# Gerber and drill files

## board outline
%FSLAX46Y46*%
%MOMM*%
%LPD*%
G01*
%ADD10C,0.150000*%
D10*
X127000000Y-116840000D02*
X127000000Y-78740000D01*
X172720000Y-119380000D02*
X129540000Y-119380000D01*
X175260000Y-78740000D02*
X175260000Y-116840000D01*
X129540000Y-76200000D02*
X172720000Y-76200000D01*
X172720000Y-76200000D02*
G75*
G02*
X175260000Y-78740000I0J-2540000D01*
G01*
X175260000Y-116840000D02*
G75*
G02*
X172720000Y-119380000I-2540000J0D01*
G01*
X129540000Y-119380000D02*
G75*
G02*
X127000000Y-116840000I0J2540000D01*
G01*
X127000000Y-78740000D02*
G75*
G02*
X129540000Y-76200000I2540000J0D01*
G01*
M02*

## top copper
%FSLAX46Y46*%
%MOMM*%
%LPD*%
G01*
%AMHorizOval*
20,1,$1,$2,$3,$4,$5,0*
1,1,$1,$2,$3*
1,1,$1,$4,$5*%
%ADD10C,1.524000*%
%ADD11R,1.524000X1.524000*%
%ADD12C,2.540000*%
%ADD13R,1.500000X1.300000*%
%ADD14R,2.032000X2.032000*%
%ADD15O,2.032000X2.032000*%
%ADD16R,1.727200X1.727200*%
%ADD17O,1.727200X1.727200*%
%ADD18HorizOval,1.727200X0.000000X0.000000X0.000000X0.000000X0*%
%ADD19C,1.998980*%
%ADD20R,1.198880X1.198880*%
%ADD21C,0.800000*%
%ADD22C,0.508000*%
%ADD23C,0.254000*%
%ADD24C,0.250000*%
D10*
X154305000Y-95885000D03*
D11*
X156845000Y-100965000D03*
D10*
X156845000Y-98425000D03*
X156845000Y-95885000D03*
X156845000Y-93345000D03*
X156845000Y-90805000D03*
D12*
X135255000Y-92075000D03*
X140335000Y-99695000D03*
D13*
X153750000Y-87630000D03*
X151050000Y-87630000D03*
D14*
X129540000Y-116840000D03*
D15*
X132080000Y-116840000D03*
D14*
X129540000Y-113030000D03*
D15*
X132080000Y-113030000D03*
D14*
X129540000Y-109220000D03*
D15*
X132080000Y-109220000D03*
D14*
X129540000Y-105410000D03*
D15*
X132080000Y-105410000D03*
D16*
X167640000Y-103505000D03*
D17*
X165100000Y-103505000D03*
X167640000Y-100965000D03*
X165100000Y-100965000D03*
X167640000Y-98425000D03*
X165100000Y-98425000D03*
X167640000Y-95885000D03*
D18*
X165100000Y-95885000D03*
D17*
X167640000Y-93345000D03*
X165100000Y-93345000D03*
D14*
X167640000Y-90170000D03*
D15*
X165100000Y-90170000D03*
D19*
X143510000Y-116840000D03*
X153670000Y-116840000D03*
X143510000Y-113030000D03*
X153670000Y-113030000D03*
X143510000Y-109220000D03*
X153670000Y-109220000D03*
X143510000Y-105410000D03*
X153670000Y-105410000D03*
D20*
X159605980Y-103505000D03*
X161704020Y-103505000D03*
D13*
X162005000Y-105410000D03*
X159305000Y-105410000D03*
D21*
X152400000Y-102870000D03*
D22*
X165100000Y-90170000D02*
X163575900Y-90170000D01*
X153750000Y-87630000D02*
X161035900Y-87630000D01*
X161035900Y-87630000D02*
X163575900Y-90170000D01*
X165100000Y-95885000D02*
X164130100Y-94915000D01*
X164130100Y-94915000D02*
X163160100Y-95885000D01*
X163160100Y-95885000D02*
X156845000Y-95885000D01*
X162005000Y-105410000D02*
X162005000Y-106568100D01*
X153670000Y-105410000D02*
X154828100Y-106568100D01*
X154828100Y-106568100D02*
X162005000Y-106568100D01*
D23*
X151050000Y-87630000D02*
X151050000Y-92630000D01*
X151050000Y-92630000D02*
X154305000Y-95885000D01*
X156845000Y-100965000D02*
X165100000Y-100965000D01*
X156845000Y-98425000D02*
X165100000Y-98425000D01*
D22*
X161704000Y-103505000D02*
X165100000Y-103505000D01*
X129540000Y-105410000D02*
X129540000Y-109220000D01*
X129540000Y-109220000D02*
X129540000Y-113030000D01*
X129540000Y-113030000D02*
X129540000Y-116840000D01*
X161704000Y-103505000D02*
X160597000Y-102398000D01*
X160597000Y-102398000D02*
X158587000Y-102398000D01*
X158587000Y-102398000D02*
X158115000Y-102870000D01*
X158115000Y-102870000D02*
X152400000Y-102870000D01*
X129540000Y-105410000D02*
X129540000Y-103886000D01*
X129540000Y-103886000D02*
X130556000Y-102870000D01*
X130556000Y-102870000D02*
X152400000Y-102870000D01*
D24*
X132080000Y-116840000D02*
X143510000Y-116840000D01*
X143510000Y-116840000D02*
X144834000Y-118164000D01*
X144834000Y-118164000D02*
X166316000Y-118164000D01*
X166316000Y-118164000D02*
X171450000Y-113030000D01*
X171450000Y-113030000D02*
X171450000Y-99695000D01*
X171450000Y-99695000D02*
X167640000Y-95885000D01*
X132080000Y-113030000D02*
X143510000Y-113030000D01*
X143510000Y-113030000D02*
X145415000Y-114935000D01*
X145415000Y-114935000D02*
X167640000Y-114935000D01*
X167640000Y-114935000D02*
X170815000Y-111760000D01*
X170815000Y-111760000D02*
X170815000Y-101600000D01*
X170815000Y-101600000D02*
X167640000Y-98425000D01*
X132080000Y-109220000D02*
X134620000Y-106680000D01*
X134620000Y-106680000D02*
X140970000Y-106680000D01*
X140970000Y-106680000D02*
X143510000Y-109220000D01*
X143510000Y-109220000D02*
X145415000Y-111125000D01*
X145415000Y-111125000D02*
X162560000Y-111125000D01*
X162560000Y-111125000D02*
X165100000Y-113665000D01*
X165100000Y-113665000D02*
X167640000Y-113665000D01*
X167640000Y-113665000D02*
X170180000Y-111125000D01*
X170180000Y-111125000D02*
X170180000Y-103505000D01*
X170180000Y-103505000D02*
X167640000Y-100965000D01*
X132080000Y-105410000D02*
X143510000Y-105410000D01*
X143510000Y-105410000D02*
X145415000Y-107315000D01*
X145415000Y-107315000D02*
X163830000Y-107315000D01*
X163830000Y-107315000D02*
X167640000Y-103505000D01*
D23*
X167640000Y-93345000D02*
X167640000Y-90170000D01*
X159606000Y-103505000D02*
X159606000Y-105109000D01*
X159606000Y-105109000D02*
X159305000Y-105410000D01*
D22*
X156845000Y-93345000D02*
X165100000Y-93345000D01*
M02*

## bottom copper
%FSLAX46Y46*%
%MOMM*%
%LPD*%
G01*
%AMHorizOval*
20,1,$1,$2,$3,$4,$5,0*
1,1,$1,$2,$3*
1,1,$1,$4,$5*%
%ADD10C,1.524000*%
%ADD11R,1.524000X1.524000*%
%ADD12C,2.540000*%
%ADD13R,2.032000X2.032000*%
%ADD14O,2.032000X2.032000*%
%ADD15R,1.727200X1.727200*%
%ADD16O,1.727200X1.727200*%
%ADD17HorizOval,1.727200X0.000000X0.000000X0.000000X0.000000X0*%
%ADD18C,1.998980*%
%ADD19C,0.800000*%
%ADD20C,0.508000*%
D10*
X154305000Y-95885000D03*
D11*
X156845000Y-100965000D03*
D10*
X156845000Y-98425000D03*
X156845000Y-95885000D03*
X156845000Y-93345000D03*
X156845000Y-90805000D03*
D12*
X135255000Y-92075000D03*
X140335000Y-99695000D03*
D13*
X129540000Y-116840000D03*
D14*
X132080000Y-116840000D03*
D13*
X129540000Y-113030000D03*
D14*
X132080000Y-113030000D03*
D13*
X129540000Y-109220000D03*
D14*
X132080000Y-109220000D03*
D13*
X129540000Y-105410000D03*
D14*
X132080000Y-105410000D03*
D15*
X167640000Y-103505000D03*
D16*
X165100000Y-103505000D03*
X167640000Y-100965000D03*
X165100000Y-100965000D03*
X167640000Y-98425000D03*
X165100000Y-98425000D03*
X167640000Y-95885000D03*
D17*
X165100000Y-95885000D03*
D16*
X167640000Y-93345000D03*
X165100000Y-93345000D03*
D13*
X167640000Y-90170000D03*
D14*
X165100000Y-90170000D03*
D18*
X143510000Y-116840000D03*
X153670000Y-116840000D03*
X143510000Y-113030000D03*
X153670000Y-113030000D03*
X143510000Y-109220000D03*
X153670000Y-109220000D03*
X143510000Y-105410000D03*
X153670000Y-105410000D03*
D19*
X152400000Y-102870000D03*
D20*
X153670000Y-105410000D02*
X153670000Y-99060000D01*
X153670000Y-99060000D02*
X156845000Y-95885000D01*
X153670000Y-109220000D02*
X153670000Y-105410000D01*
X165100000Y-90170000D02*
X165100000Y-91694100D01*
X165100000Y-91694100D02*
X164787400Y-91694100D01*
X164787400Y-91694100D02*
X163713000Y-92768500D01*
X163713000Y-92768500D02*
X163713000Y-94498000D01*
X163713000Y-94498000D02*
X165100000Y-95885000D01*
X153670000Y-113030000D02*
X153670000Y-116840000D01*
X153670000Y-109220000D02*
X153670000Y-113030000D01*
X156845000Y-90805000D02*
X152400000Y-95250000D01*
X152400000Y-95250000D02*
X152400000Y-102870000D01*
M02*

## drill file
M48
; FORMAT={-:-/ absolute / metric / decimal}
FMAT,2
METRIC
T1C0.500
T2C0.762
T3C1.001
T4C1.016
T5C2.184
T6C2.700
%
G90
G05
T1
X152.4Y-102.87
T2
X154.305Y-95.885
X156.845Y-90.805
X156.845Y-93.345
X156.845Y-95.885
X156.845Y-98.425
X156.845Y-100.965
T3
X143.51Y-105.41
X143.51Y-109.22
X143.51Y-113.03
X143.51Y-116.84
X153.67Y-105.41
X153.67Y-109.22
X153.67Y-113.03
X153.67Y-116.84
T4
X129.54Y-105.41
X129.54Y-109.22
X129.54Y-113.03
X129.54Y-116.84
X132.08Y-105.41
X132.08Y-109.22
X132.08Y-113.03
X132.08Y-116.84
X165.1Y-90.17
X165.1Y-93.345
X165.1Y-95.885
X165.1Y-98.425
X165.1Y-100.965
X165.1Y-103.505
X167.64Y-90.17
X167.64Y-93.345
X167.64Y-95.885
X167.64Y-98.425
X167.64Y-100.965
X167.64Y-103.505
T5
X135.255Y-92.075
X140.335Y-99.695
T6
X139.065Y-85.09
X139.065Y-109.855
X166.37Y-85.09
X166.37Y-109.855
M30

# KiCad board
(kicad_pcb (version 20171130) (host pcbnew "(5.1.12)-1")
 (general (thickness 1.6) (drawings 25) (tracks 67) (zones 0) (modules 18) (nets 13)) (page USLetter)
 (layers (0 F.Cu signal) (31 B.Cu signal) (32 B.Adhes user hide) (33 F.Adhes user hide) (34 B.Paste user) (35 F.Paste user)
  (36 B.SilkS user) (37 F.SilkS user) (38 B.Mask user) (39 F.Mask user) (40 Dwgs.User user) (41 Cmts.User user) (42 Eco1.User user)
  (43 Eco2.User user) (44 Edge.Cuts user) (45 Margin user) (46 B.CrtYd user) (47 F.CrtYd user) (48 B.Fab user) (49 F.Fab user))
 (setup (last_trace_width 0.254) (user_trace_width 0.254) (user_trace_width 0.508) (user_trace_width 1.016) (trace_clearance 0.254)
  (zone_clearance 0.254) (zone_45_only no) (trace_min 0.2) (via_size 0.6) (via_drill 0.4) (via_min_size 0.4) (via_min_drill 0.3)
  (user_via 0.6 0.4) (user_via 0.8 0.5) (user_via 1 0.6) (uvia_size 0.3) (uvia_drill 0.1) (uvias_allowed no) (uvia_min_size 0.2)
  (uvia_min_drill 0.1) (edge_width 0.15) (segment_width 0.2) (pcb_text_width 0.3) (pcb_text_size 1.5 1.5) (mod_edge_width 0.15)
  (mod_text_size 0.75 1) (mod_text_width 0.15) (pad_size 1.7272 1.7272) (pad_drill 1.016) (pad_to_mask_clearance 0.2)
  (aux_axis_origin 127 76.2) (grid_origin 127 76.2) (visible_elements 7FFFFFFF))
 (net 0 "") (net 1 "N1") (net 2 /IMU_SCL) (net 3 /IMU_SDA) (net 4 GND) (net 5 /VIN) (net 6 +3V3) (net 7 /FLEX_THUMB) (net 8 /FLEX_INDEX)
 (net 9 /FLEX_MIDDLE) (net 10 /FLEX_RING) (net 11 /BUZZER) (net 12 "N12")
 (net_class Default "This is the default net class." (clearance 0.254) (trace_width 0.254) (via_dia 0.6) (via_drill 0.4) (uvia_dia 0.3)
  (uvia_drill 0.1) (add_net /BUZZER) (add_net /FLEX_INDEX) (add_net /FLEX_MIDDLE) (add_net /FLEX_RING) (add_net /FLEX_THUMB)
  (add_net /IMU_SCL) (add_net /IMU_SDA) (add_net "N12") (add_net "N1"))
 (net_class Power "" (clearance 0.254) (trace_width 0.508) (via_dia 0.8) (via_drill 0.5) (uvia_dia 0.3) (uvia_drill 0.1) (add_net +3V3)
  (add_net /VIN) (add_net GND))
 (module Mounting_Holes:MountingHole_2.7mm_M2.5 (layer F.Cu) (at 139.065 109.855)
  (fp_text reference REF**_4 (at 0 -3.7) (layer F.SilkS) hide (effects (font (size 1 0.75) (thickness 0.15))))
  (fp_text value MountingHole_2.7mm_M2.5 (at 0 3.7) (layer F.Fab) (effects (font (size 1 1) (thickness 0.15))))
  (pad 1 np_thru_hole circle (at 0 0) (size 2.7 2.7) (drill 2.7) (layers *.Cu *.Mask F.SilkS)))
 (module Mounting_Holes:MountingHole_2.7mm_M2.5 (layer F.Cu) (at 166.37 109.855)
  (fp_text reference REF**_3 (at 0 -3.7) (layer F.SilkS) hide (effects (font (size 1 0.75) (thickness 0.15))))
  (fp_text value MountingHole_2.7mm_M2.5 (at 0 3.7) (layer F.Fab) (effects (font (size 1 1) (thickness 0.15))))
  (pad 1 np_thru_hole circle (at 0 0) (size 2.7 2.7) (drill 2.7) (layers *.Cu *.Mask F.SilkS)))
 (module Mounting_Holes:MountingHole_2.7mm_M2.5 (layer F.Cu) (at 166.37 85.09)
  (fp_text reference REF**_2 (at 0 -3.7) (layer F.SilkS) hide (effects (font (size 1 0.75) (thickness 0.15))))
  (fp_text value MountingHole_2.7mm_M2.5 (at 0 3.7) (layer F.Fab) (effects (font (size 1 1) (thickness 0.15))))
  (pad 1 np_thru_hole circle (at 0 0) (size 2.7 2.7) (drill 2.7) (layers *.Cu *.Mask F.SilkS)))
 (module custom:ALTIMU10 (layer F.Cu) (at 156.845 95.885 90)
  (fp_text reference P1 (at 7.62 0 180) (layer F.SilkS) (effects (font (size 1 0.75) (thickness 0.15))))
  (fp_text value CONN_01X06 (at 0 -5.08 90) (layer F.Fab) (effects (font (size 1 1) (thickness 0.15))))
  (pad 6 thru_hole circle (at 0 -2.54 90) (size 1.524 1.524) (drill 0.762) (layers *.Cu *.Mask F.SilkS) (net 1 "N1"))
  (pad 1 thru_hole rect (at -5.08 0 90) (size 1.524 1.524) (drill 0.762) (layers *.Cu *.Mask F.SilkS) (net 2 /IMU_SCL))
  (pad 2 thru_hole circle (at -2.54 0 90) (size 1.524 1.524) (drill 0.762) (layers *.Cu *.Mask F.SilkS) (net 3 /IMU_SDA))
  (pad 3 thru_hole circle (at 0 0 90) (size 1.524 1.524) (drill 0.762) (layers *.Cu *.Mask F.SilkS) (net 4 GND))
  (pad 4 thru_hole circle (at 2.54 0 90) (size 1.524 1.524) (drill 0.762) (layers *.Cu *.Mask F.SilkS) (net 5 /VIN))
  (pad 5 thru_hole circle (at 5.08 0 90) (size 1.524 1.524) (drill 0.762) (layers *.Cu *.Mask F.SilkS) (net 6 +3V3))
  (pad "" np_thru_hole circle (at 3.81 -21.59 90) (size 2.54 2.54) (drill 2.1844) (layers *.Cu *.Mask F.SilkS))
  (pad "" np_thru_hole circle (at -3.81 -16.51 90) (size 2.54 2.54) (drill 2.1844) (layers *.Cu *.Mask F.SilkS)))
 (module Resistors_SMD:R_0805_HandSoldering (layer F.Cu) (at 152.4 87.63 180)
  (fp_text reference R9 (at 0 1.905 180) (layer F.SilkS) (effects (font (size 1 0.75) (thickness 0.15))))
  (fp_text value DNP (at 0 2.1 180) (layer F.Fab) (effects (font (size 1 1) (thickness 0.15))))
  (pad 1 smd rect (at -1.35 0 180) (size 1.5 1.3) (layers F.Cu F.Paste F.Mask) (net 4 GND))
  (pad 2 smd rect (at 1.35 0 180) (size 1.5 1.3) (layers F.Cu F.Paste F.Mask) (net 1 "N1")))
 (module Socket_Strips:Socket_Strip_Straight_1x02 (layer F.Cu) (at 129.54 116.84)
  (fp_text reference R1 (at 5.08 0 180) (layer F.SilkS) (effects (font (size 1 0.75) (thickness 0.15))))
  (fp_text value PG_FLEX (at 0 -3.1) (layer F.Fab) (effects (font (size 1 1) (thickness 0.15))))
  (pad 1 thru_hole rect (at 0 0) (size 2.032 2.032) (drill 1.016) (layers *.Cu *.Mask F.SilkS) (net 6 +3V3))
  (pad 2 thru_hole oval (at 2.54 0) (size 2.032 2.032) (drill 1.016) (layers *.Cu *.Mask F.SilkS) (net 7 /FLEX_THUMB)))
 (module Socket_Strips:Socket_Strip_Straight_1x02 (layer F.Cu) (at 129.54 113.03)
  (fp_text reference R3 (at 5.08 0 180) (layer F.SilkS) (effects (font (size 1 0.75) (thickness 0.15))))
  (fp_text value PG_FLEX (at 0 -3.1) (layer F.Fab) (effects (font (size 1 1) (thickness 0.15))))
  (pad 1 thru_hole rect (at 0 0) (size 2.032 2.032) (drill 1.016) (layers *.Cu *.Mask F.SilkS) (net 6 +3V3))
  (pad 2 thru_hole oval (at 2.54 0) (size 2.032 2.032) (drill 1.016) (layers *.Cu *.Mask F.SilkS) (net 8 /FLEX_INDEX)))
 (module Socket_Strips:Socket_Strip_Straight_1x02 (layer F.Cu) (at 129.54 109.22)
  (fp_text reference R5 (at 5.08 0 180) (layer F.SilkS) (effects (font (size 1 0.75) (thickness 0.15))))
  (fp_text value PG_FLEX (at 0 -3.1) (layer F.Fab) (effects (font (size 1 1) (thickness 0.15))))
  (pad 1 thru_hole rect (at 0 0) (size 2.032 2.032) (drill 1.016) (layers *.Cu *.Mask F.SilkS) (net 6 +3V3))
  (pad 2 thru_hole oval (at 2.54 0) (size 2.032 2.032) (drill 1.016) (layers *.Cu *.Mask F.SilkS) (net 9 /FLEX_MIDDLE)))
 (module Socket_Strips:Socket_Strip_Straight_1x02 (layer F.Cu) (at 129.54 105.41)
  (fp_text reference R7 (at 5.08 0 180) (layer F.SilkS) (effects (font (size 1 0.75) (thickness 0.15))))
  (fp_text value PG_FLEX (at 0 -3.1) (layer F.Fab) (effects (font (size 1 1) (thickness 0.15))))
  (pad 1 thru_hole rect (at 0 0) (size 2.032 2.032) (drill 1.016) (layers *.Cu *.Mask F.SilkS) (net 6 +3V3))
  (pad 2 thru_hole oval (at 2.54 0) (size 2.032 2.032) (drill 1.016) (layers *.Cu *.Mask F.SilkS) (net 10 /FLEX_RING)))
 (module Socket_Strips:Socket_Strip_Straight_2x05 (layer B.Cu) (at 167.64 103.505 90)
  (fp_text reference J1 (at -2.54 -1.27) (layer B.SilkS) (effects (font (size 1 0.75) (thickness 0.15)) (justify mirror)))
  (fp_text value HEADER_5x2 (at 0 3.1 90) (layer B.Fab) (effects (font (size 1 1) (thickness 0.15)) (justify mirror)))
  (pad 1 thru_hole rect (at 0 0 90) (size 1.7272 1.7272) (drill 1.016) (layers *.Cu *.Mask B.SilkS) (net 10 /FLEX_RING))
  (pad 2 thru_hole oval (at 0 -2.54 90) (size 1.7272 1.7272) (drill 1.016) (layers *.Cu *.Mask B.SilkS) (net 6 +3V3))
  (pad 3 thru_hole oval (at 2.54 0 90) (size 1.7272 1.7272) (drill 1.016) (layers *.Cu *.Mask B.SilkS) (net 9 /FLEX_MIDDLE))
  (pad 4 thru_hole oval (at 2.54 -2.54 90) (size 1.7272 1.7272) (drill 1.016) (layers *.Cu *.Mask B.SilkS) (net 2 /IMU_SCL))
  (pad 5 thru_hole oval (at 5.08 0 90) (size 1.7272 1.7272) (drill 1.016) (layers *.Cu *.Mask B.SilkS) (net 8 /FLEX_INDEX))
  (pad 6 thru_hole oval (at 5.08 -2.54 90) (size 1.7272 1.7272) (drill 1.016) (layers *.Cu *.Mask B.SilkS) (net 3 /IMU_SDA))
  (pad 7 thru_hole oval (at 7.62 0 90) (size 1.7272 1.7272) (drill 1.016) (layers *.Cu *.Mask B.SilkS) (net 7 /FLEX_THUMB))
  (pad 8 thru_hole oval (at 7.62 -2.54 45) (size 1.7272 1.7272) (drill 1.016) (layers *.Cu *.Mask B.SilkS) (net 4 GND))
  (pad 9 thru_hole oval (at 10.16 0 90) (size 1.7272 1.7272) (drill 1.016) (layers *.Cu *.Mask B.SilkS) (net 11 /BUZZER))
  (pad 10 thru_hole oval (at 10.16 -2.54 90) (size 1.7272 1.7272) (drill 1.016) (layers *.Cu *.Mask B.SilkS) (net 5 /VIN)))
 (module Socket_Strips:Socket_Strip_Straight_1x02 (layer F.Cu) (at 167.64 90.17 180)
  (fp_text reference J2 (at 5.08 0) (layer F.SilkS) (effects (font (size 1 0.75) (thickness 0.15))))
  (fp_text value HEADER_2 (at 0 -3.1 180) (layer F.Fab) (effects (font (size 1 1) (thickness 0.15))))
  (pad 1 thru_hole rect (at 0 0 180) (size 2.032 2.032) (drill 1.016) (layers *.Cu *.Mask F.SilkS) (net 11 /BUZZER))
  (pad 2 thru_hole oval (at 2.54 0 180) (size 2.032 2.032) (drill 1.016) (layers *.Cu *.Mask F.SilkS) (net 4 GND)))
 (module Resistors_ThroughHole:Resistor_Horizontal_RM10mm (layer F.Cu) (at 143.51 116.84)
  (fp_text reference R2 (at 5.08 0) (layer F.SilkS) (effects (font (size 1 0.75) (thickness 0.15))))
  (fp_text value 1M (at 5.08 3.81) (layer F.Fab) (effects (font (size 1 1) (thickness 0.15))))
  (pad 1 thru_hole circle (at 0 0) (size 1.99898 1.99898) (drill 1.00076) (layers *.Cu *.SilkS *.Mask) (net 7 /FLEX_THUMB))
  (pad 2 thru_hole circle (at 10.16 0) (size 1.99898 1.99898) (drill 1.00076) (layers *.Cu *.SilkS *.Mask) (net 4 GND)))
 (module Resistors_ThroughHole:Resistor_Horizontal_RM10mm (layer F.Cu) (at 143.51 113.03)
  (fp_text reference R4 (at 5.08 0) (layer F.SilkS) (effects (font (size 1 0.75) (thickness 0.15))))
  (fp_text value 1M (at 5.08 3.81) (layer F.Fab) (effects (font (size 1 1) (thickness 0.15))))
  (pad 1 thru_hole circle (at 0 0) (size 1.99898 1.99898) (drill 1.00076) (layers *.Cu *.SilkS *.Mask) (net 8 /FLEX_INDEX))
  (pad 2 thru_hole circle (at 10.16 0) (size 1.99898 1.99898) (drill 1.00076) (layers *.Cu *.SilkS *.Mask) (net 4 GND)))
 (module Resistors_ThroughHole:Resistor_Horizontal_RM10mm (layer F.Cu) (at 143.51 109.22)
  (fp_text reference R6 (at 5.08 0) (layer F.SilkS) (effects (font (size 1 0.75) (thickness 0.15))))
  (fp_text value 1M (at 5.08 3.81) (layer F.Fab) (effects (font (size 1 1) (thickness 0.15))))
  (pad 1 thru_hole circle (at 0 0) (size 1.99898 1.99898) (drill 1.00076) (layers *.Cu *.SilkS *.Mask) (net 9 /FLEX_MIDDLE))
  (pad 2 thru_hole circle (at 10.16 0) (size 1.99898 1.99898) (drill 1.00076) (layers *.Cu *.SilkS *.Mask) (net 4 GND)))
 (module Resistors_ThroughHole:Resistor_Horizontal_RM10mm (layer F.Cu) (at 143.51 105.41)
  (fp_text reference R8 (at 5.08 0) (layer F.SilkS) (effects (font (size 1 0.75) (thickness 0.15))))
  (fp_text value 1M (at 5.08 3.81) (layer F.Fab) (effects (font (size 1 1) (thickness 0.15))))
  (pad 1 thru_hole circle (at 0 0) (size 1.99898 1.99898) (drill 1.00076) (layers *.Cu *.SilkS *.Mask) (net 10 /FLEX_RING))
  (pad 2 thru_hole circle (at 10.16 0) (size 1.99898 1.99898) (drill 1.00076) (layers *.Cu *.SilkS *.Mask) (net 4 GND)))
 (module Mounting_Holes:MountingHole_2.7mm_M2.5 (layer F.Cu) (at 139.065 85.09)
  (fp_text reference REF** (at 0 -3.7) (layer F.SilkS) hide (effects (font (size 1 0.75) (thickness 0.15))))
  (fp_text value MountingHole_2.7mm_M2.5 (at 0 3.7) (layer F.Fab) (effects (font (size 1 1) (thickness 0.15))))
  (pad 1 np_thru_hole circle (at 0 0) (size 2.7 2.7) (drill 2.7) (layers *.Cu *.Mask F.SilkS)))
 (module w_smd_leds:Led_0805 (layer F.Cu) (at 160.655 103.505)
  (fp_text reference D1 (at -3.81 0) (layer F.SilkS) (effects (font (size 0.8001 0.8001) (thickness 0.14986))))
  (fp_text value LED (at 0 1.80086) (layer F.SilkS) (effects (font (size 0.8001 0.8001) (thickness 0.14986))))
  (pad 1 smd rect (at -1.04902 0) (size 1.19888 1.19888) (layers F.Cu F.Paste F.Mask) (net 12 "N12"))
  (pad 2 smd rect (at 1.04902 0) (size 1.19888 1.19888) (layers F.Cu F.Paste F.Mask) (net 6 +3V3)))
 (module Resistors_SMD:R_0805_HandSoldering (layer F.Cu) (at 160.655 105.41 180)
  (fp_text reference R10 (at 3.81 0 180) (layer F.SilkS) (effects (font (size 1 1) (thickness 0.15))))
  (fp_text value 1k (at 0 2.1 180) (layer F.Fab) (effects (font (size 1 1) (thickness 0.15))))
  (pad 1 smd rect (at -1.35 0 180) (size 1.5 1.3) (layers F.Cu F.Paste F.Mask) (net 4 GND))
  (pad 2 smd rect (at 1.35 0 180) (size 1.5 1.3) (layers F.Cu F.Paste F.Mask) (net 12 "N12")))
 (gr_line (start 127 116.84) (end 127 78.74) (layer Edge.Cuts) (width 0.15))
 (gr_line (start 172.72 119.38) (end 129.54 119.38) (layer Edge.Cuts) (width 0.15))
 (gr_line (start 175.26 78.74) (end 175.26 116.84) (layer Edge.Cuts) (width 0.15))
 (gr_line (start 129.54 76.2) (end 172.72 76.2) (layer Edge.Cuts) (width 0.15))
 (gr_arc (start 172.72 78.74) (end 172.72 76.2) (angle 90) (layer Edge.Cuts) (width 0.15))
 (gr_arc (start 172.72 116.84) (end 175.26 116.84) (angle 90) (layer Edge.Cuts) (width 0.15))
 (gr_arc (start 129.54 116.84) (end 129.54 119.38) (angle 90) (layer Edge.Cuts) (width 0.15))
 (gr_arc (start 129.54 78.74) (end 127 78.74) (angle 90) (layer Edge.Cuts) (width 0.15))
 (segment (start 165.1 90.17) (end 163.5759 90.17) (width 0.508) (layer F.Cu) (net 4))
 (segment (start 153.75 87.63) (end 161.0359 87.63) (width 0.508) (layer F.Cu) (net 4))
 (segment (start 161.0359 87.63) (end 163.5759 90.17) (width 0.508) (layer F.Cu) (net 4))
 (segment (start 153.67 105.41) (end 153.67 99.06) (width 0.508) (layer B.Cu) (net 4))
 (segment (start 153.67 99.06) (end 156.845 95.885) (width 0.508) (layer B.Cu) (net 4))
 (segment (start 153.67 109.22) (end 153.67 105.41) (width 0.508) (layer B.Cu) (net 4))
 (segment (start 165.1 90.17) (end 165.1 91.6941) (width 0.508) (layer B.Cu) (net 4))
 (segment (start 165.1 91.6941) (end 164.7874 91.6941) (width 0.508) (layer B.Cu) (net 4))
 (segment (start 164.7874 91.6941) (end 163.713 92.7685) (width 0.508) (layer B.Cu) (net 4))
 (segment (start 163.713 92.7685) (end 163.713 94.498) (width 0.508) (layer B.Cu) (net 4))
 (segment (start 163.713 94.498) (end 165.1 95.885) (width 0.508) (layer B.Cu) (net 4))
 (segment (start 165.1 95.885) (end 164.1301 94.915) (width 0.508) (layer F.Cu) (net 4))
 (segment (start 164.1301 94.915) (end 163.1601 95.885) (width 0.508) (layer F.Cu) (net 4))
 (segment (start 163.1601 95.885) (end 156.845 95.885) (width 0.508) (layer F.Cu) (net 4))
 (segment (start 162.005 105.41) (end 162.005 106.5681) (width 0.508) (layer F.Cu) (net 4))
 (segment (start 153.67 105.41) (end 154.8281 106.5681) (width 0.508) (layer F.Cu) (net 4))
 (segment (start 154.8281 106.5681) (end 162.005 106.5681) (width 0.508) (layer F.Cu) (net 4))
 (segment (start 153.67 113.03) (end 153.67 116.84) (width 0.508) (layer B.Cu) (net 4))
 (segment (start 153.67 109.22) (end 153.67 113.03) (width 0.508) (layer B.Cu) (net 4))
 (segment (start 151.05 87.63) (end 151.05 92.63) (width 0.254) (layer F.Cu) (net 1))
 (segment (start 151.05 92.63) (end 154.305 95.885) (width 0.254) (layer F.Cu) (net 1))
 (segment (start 156.845 100.965) (end 165.1 100.965) (width 0.254) (layer F.Cu) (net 2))
 (segment (start 156.845 98.425) (end 165.1 98.425) (width 0.254) (layer F.Cu) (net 3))
 (segment (start 161.704 103.505) (end 165.1 103.505) (width 0.508) (layer F.Cu) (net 6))
 (segment (start 129.54 105.41) (end 129.54 109.22) (width 0.508) (layer F.Cu) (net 6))
 (segment (start 129.54 109.22) (end 129.54 113.03) (width 0.508) (layer F.Cu) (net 6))
 (segment (start 129.54 113.03) (end 129.54 116.84) (width 0.508) (layer F.Cu) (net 6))
 (segment (start 156.845 90.805) (end 152.4 95.25) (width 0.508) (layer B.Cu) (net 6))
 (segment (start 152.4 95.25) (end 152.4 102.87) (width 0.508) (layer B.Cu) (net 6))
 (segment (start 161.704 103.505) (end 160.597 102.398) (width 0.508) (layer F.Cu) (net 6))
 (segment (start 160.597 102.398) (end 158.587 102.398) (width 0.508) (layer F.Cu) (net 6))
 (segment (start 158.587 102.398) (end 158.115 102.87) (width 0.508) (layer F.Cu) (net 6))
 (segment (start 158.115 102.87) (end 152.4 102.87) (width 0.508) (layer F.Cu) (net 6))
 (segment (start 129.54 105.41) (end 129.54 103.886) (width 0.508) (layer F.Cu) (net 6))
 (segment (start 129.54 103.886) (end 130.556 102.87) (width 0.508) (layer F.Cu) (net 6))
 (segment (start 130.556 102.87) (end 152.4 102.87) (width 0.508) (layer F.Cu) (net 6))
 (via (at 152.4 102.87) (size 0.8) (drill 0.5) (layers F.Cu B.Cu) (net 6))
 (segment (start 132.08 116.84) (end 143.51 116.84) (width 0.25) (layer F.Cu) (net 7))
 (segment (start 143.51 116.84) (end 144.834 118.164) (width 0.25) (layer F.Cu) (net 7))
 (segment (start 144.834 118.164) (end 166.316 118.164) (width 0.25) (layer F.Cu) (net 7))
 (segment (start 166.316 118.164) (end 171.45 113.03) (width 0.25) (layer F.Cu) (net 7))
 (segment (start 171.45 113.03) (end 171.45 99.695) (width 0.25) (layer F.Cu) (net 7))
 (segment (start 171.45 99.695) (end 167.64 95.885) (width 0.25) (layer F.Cu) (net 7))
 (segment (start 132.08 113.03) (end 143.51 113.03) (width 0.25) (layer F.Cu) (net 8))
 (segment (start 143.51 113.03) (end 145.415 114.935) (width 0.25) (layer F.Cu) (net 8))
 (segment (start 145.415 114.935) (end 167.64 114.935) (width 0.25) (layer F.Cu) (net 8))
 (segment (start 167.64 114.935) (end 170.815 111.76) (width 0.25) (layer F.Cu) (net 8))
 (segment (start 170.815 111.76) (end 170.815 101.6) (width 0.25) (layer F.Cu) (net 8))
 (segment (start 170.815 101.6) (end 167.64 98.425) (width 0.25) (layer F.Cu) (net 8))
 (segment (start 132.08 109.22) (end 134.62 106.68) (width 0.25) (layer F.Cu) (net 9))
 (segment (start 134.62 106.68) (end 140.97 106.68) (width 0.25) (layer F.Cu) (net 9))
 (segment (start 140.97 106.68) (end 143.51 109.22) (width 0.25) (layer F.Cu) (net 9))
 (segment (start 143.51 109.22) (end 145.415 111.125) (width 0.25) (layer F.Cu) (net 9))
 (segment (start 145.415 111.125) (end 162.56 111.125) (width 0.25) (layer F.Cu) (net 9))
 (segment (start 162.56 111.125) (end 165.1 113.665) (width 0.25) (layer F.Cu) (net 9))
 (segment (start 165.1 113.665) (end 167.64 113.665) (width 0.25) (layer F.Cu) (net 9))
 (segment (start 167.64 113.665) (end 170.18 111.125) (width 0.25) (layer F.Cu) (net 9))
 (segment (start 170.18 111.125) (end 170.18 103.505) (width 0.25) (layer F.Cu) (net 9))
 (segment (start 170.18 103.505) (end 167.64 100.965) (width 0.25) (layer F.Cu) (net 9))
 (segment (start 132.08 105.41) (end 143.51 105.41) (width 0.25) (layer F.Cu) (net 10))
 (segment (start 143.51 105.41) (end 145.415 107.315) (width 0.25) (layer F.Cu) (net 10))
 (segment (start 145.415 107.315) (end 163.83 107.315) (width 0.25) (layer F.Cu) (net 10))
 (segment (start 163.83 107.315) (end 167.64 103.505) (width 0.25) (layer F.Cu) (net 10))
 (segment (start 167.64 93.345) (end 167.64 90.17) (width 0.254) (layer F.Cu) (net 11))
 (segment (start 159.606 103.505) (end 159.606 105.109) (width 0.254) (layer F.Cu) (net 12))
 (segment (start 159.606 105.109) (end 159.305 105.41) (width 0.254) (layer F.Cu) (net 12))
 (segment (start 156.845 93.345) (end 165.1 93.345) (width 0.508) (layer F.Cu) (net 5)))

